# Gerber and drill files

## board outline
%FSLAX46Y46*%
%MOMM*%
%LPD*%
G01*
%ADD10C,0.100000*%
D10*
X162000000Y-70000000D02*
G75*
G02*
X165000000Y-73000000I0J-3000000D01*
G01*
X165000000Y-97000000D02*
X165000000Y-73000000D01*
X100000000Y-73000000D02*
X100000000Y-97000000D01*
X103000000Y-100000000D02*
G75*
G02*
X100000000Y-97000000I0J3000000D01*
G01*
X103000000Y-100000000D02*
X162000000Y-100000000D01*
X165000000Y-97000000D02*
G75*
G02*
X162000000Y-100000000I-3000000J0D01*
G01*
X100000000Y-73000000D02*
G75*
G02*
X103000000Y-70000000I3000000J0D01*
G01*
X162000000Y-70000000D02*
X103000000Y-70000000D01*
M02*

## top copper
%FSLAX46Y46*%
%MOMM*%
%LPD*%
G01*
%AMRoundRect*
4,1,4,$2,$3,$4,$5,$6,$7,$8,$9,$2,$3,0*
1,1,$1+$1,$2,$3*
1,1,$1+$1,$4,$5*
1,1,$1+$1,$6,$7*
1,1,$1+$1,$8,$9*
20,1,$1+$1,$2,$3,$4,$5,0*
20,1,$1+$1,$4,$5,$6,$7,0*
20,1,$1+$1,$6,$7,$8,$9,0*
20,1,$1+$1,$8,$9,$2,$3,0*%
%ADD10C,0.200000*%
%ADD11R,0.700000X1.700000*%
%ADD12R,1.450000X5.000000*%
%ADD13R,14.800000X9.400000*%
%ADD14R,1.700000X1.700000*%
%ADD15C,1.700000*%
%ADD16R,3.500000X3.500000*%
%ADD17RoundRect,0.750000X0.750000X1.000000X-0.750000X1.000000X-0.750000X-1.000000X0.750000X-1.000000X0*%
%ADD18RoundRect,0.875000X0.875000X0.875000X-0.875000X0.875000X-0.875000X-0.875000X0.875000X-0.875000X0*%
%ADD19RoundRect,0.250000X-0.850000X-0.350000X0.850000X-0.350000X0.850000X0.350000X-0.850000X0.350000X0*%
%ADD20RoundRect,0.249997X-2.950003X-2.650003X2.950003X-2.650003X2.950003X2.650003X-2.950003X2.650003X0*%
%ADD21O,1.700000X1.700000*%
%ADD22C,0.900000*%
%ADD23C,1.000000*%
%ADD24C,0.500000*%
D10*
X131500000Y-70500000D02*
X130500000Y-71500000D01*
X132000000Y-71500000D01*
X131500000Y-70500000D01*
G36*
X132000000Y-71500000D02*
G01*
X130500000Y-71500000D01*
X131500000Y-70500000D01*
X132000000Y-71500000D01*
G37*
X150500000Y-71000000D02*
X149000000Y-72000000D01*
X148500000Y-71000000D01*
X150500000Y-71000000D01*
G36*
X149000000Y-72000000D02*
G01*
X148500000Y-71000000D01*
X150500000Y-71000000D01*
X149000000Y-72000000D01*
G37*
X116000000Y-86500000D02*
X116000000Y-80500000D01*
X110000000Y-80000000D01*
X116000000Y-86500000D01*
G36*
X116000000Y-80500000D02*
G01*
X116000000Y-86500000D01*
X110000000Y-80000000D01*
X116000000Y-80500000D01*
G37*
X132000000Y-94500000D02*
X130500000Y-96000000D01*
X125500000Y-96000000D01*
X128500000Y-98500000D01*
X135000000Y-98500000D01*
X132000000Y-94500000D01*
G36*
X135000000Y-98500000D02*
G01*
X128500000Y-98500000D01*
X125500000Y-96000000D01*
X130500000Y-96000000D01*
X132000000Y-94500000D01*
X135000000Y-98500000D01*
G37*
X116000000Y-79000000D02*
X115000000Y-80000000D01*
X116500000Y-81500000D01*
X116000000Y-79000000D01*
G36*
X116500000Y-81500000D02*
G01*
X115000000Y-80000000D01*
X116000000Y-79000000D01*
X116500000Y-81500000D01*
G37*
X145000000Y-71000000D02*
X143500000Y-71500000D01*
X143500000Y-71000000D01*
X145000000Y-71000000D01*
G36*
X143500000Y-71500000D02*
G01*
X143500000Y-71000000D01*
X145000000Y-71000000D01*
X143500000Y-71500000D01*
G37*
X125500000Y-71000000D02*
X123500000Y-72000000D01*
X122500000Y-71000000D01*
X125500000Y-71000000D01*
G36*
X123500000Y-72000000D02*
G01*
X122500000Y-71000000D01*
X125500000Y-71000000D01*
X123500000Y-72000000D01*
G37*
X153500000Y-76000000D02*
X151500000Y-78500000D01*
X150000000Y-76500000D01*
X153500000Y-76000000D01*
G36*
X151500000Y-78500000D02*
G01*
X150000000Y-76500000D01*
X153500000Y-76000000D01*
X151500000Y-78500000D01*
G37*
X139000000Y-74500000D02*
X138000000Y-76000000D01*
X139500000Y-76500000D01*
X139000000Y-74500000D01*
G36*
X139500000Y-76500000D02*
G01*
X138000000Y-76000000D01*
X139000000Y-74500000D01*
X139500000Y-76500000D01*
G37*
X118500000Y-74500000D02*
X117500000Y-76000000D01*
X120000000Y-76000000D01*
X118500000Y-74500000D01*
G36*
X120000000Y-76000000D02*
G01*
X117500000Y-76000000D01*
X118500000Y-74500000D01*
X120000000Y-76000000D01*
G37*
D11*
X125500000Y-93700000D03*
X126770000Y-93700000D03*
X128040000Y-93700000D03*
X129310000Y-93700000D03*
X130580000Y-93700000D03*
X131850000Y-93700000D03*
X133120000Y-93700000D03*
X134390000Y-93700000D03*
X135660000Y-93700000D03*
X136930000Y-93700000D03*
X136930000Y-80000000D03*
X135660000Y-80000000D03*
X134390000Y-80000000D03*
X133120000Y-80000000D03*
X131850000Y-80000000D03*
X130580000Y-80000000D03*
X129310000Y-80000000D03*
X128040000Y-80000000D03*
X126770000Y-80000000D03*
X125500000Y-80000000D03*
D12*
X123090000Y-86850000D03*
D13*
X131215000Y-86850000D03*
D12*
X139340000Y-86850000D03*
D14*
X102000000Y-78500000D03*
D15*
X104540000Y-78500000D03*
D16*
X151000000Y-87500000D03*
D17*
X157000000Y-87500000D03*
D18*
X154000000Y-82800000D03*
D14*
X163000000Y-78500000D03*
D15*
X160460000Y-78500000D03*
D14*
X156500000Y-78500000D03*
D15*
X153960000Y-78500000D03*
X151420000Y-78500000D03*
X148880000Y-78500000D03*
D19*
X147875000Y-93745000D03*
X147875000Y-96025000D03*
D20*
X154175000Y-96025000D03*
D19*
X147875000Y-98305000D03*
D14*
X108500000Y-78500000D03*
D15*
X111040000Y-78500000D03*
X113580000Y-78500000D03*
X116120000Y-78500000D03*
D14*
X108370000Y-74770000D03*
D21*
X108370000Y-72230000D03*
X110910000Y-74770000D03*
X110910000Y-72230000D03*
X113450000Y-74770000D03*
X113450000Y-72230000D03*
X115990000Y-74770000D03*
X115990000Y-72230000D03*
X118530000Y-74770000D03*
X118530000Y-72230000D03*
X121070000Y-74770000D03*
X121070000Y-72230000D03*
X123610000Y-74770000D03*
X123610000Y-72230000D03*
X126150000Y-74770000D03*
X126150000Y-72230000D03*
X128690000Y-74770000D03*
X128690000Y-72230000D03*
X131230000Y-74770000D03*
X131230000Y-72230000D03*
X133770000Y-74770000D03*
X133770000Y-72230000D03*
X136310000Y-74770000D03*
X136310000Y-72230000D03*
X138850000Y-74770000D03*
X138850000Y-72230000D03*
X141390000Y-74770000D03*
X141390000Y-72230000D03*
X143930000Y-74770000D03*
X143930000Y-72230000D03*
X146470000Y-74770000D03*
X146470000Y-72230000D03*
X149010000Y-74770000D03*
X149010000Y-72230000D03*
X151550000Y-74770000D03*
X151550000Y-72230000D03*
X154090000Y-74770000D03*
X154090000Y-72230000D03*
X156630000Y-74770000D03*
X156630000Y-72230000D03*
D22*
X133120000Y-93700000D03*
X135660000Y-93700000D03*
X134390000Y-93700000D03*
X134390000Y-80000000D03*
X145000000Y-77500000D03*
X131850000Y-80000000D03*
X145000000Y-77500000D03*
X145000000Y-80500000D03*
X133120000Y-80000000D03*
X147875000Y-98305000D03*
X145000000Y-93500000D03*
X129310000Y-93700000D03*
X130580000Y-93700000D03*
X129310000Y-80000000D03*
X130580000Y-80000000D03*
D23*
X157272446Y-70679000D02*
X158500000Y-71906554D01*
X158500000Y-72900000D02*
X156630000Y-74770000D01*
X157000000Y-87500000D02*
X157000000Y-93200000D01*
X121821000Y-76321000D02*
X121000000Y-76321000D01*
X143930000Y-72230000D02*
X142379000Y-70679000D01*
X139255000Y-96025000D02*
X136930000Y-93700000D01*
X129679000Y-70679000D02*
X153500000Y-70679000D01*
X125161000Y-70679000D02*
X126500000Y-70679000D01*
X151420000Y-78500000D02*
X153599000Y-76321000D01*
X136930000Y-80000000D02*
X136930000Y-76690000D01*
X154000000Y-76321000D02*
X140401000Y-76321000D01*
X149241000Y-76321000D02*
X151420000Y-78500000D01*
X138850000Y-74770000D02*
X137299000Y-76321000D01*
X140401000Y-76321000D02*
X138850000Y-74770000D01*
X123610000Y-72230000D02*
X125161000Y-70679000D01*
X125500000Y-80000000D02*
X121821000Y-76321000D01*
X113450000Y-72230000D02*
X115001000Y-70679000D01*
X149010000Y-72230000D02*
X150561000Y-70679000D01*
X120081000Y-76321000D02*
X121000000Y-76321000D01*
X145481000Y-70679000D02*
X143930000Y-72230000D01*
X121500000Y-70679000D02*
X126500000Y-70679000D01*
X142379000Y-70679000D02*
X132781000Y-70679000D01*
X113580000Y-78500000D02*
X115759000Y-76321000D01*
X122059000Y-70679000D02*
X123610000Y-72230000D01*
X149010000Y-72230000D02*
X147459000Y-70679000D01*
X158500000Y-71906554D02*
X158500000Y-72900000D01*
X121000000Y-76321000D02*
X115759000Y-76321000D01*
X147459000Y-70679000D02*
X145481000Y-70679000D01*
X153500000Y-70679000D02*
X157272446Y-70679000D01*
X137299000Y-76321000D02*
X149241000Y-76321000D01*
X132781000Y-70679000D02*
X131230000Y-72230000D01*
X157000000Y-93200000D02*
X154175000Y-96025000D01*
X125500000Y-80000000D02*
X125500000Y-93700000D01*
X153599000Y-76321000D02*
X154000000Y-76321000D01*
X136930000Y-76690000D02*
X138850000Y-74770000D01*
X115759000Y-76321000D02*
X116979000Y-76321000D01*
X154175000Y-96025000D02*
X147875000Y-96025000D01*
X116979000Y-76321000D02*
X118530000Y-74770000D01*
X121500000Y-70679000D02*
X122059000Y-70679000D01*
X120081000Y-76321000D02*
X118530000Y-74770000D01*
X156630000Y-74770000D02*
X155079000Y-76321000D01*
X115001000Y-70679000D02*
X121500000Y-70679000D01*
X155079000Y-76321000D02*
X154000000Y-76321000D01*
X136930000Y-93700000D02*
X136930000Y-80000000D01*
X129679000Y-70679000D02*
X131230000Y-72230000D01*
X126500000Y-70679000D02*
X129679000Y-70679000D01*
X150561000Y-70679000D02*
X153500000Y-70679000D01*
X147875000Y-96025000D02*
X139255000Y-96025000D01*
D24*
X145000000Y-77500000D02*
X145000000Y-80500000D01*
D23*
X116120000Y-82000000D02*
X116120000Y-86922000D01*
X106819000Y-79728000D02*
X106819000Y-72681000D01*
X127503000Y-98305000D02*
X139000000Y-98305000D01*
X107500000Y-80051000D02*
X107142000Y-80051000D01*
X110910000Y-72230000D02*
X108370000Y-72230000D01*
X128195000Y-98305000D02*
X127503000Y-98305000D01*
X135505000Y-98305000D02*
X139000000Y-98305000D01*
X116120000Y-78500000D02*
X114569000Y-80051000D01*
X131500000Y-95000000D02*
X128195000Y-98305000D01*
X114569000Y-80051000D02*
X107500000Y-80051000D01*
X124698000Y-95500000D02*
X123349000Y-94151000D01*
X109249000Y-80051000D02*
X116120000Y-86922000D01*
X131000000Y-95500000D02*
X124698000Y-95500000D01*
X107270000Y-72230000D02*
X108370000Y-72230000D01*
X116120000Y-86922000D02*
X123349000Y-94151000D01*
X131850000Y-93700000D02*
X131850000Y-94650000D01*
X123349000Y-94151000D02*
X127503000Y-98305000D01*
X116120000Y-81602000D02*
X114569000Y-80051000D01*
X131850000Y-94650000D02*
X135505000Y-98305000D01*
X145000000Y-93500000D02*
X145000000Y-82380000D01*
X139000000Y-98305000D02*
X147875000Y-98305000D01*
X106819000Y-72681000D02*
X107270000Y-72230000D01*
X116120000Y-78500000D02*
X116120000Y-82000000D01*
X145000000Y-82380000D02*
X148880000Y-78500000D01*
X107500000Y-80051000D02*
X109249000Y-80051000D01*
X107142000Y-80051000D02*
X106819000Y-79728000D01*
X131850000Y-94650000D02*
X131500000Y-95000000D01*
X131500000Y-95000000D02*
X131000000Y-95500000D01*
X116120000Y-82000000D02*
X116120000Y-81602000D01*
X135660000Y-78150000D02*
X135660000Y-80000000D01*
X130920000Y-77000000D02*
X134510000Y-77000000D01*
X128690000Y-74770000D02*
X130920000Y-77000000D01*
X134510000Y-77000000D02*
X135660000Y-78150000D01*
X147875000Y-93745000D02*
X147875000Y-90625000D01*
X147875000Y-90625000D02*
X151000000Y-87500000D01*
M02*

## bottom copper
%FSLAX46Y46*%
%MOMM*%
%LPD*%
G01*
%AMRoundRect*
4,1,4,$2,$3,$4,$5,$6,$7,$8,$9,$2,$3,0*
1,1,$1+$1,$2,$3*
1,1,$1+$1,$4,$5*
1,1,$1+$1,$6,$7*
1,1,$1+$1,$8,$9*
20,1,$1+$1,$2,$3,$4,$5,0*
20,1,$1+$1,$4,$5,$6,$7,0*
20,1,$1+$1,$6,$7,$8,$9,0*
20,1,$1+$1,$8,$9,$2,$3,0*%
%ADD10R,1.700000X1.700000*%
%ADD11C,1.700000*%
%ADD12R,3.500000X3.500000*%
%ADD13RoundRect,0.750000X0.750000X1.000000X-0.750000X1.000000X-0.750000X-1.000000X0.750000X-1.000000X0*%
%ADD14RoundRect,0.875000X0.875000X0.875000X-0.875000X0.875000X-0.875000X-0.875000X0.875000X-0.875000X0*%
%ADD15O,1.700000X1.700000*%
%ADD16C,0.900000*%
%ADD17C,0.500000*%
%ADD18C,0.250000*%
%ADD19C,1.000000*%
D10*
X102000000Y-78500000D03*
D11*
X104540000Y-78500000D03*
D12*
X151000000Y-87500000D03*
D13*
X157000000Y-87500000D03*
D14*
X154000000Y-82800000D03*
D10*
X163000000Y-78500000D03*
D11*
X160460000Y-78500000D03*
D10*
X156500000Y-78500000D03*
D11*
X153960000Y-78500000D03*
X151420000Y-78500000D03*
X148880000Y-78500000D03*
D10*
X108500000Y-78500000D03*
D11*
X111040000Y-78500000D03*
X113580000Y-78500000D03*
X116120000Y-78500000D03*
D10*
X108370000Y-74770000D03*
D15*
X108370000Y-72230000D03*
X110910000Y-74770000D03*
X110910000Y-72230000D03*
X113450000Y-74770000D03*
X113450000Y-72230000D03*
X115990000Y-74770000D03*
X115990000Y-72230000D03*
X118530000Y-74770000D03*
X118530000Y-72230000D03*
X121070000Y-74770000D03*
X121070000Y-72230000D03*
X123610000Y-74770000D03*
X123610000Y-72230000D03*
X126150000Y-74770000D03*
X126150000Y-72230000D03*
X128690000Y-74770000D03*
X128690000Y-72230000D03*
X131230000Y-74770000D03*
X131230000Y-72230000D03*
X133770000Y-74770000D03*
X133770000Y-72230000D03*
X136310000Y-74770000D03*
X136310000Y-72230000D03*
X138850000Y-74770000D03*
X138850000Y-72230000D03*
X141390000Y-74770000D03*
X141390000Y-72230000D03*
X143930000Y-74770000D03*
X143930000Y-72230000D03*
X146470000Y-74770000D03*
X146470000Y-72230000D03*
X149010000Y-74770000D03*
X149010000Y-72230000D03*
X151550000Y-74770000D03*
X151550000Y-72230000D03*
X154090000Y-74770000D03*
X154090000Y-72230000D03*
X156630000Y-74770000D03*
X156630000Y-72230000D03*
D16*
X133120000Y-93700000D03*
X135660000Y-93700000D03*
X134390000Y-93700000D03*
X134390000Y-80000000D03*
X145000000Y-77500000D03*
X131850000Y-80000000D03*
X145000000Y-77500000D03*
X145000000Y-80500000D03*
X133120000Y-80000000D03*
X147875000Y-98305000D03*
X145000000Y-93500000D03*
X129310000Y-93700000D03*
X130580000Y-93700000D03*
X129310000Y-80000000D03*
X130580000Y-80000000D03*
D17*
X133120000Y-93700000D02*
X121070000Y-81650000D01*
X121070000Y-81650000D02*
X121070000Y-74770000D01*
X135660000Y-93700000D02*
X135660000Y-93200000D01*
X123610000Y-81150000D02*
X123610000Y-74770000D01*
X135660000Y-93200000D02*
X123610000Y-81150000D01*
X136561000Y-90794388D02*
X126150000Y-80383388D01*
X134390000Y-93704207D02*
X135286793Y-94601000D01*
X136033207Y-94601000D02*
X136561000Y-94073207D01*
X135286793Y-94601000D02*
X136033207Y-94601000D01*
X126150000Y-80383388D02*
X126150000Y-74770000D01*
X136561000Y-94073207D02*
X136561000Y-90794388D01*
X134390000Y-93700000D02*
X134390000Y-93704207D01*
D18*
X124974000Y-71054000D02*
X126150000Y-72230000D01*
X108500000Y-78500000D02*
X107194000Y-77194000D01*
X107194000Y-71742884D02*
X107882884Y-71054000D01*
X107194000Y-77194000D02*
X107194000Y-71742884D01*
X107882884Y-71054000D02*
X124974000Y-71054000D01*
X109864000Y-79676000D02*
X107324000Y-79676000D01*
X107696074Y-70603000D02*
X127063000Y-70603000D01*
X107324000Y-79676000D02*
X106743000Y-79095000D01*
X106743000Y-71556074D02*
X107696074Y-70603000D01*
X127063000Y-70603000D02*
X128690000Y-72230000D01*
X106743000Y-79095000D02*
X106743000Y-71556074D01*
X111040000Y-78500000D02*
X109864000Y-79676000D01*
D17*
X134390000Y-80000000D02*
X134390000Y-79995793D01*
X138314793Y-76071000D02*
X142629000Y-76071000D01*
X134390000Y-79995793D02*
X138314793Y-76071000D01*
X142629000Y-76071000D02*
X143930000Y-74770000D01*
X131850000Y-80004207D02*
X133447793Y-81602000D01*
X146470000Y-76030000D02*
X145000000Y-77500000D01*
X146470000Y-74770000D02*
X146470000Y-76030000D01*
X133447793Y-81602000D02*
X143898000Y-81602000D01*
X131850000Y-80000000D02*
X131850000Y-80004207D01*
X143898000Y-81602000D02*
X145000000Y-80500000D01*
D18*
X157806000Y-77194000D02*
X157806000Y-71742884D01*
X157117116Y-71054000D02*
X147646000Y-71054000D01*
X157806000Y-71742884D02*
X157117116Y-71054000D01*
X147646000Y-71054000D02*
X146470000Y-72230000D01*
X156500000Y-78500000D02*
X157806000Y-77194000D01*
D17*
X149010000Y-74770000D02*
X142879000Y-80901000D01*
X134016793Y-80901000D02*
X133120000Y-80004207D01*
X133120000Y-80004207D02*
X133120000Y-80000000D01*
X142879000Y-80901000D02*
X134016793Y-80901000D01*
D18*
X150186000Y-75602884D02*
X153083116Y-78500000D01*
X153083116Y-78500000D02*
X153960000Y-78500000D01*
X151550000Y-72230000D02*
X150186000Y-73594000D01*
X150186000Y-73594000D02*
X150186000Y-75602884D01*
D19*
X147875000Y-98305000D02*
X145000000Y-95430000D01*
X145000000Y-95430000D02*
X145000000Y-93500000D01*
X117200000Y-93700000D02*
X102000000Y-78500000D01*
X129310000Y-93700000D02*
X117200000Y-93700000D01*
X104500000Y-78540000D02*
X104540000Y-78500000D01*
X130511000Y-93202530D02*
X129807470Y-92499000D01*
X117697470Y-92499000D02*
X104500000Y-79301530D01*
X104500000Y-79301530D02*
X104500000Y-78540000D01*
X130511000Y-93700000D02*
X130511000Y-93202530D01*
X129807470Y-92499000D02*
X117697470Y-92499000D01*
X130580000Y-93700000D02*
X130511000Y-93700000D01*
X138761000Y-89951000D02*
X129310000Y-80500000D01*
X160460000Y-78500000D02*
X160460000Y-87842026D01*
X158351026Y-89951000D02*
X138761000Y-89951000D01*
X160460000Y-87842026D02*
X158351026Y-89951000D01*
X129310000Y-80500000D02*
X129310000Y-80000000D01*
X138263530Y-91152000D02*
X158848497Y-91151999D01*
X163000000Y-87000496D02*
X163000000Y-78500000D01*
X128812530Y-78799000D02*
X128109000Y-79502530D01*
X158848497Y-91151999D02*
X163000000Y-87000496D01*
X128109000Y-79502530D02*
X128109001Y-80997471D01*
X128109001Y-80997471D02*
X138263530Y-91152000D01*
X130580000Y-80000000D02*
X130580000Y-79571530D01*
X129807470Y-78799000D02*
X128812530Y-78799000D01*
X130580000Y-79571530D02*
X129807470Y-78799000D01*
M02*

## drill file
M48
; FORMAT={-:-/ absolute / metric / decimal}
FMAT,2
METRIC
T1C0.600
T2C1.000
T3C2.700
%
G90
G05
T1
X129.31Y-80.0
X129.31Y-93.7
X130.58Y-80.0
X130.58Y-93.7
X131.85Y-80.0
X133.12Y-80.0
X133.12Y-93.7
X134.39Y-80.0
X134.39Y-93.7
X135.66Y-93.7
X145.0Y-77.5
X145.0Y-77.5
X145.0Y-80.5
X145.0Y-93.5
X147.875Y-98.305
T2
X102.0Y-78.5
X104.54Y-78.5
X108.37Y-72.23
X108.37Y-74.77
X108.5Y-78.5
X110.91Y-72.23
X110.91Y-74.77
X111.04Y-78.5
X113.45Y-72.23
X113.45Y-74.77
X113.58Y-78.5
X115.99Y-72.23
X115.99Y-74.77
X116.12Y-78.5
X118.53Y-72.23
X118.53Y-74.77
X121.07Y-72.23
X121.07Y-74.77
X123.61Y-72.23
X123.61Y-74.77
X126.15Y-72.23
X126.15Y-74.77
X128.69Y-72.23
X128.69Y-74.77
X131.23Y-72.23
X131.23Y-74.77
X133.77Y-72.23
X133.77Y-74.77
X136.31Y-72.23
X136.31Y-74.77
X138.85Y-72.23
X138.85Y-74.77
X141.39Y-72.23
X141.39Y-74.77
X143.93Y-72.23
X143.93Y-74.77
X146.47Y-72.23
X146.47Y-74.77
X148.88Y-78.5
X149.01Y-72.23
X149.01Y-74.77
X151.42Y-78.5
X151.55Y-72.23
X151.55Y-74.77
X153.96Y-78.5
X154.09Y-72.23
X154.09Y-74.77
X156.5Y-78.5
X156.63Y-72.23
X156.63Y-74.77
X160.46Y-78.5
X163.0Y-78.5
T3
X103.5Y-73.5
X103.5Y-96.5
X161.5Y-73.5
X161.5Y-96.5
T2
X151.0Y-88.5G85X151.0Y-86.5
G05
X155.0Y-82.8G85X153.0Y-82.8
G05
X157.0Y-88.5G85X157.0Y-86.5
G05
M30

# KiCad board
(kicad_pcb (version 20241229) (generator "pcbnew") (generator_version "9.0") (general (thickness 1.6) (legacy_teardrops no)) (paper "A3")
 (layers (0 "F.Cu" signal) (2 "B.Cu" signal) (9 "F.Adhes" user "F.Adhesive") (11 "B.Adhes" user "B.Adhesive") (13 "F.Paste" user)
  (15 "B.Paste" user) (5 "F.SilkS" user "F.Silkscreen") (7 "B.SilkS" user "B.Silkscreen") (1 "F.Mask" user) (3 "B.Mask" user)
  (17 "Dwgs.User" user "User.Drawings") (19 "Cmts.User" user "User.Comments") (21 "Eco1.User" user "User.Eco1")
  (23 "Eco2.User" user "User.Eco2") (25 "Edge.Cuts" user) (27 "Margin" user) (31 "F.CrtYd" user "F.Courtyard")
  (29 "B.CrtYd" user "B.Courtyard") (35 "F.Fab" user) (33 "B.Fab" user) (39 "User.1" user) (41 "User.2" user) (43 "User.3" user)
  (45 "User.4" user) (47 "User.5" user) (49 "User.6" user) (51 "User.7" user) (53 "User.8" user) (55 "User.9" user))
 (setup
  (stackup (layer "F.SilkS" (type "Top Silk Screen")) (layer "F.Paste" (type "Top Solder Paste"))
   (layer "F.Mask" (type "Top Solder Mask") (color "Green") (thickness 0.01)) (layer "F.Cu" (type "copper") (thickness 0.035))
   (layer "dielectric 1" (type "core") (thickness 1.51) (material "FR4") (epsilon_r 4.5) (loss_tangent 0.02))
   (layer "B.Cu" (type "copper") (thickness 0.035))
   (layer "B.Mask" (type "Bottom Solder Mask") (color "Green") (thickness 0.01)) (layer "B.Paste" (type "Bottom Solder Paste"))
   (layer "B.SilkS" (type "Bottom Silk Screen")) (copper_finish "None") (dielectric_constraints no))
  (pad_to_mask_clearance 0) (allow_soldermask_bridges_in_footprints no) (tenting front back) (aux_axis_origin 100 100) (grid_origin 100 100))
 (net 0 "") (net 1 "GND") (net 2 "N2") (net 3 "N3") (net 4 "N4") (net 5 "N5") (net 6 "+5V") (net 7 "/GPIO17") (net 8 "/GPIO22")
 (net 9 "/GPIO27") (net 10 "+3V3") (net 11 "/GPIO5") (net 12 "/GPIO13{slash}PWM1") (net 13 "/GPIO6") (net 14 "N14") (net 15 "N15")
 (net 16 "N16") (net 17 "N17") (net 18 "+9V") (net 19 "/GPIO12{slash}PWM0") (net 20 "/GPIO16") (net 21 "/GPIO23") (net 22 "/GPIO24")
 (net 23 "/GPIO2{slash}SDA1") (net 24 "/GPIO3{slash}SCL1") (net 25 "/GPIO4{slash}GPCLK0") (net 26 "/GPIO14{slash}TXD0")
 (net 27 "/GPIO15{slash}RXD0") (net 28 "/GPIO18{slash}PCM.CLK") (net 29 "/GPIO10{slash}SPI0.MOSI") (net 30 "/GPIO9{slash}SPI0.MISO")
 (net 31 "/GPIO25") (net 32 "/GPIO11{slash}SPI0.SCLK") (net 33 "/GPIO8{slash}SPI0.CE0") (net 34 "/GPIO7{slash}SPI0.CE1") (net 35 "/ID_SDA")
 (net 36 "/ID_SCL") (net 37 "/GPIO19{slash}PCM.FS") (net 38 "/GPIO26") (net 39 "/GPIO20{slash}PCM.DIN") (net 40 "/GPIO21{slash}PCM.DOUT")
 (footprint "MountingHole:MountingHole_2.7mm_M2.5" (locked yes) (layer "F.Cu") (at 161.5 73.5)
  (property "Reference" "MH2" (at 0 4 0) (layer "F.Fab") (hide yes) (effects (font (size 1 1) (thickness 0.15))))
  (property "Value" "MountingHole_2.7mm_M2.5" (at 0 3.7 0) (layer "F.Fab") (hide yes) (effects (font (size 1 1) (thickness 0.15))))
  (pad "" np_thru_hole circle (at 0 0) (size 2.7 2.7) (drill 2.7) (layers "*.Cu" "*.Mask")))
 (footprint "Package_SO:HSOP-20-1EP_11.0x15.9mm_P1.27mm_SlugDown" (layer "F.Cu") (at 131.215 86.85 90)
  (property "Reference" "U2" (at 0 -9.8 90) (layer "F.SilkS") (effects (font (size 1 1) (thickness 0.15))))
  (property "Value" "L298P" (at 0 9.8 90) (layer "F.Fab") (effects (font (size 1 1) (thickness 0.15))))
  (pad "1" smd rect (at -6.85 -5.715 90) (size 1.7 0.7) (layers "F.Cu" "F.Mask" "F.Paste") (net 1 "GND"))
  (pad "2" smd rect (at -6.85 -4.445 90) (size 1.7 0.7) (layers "F.Cu" "F.Mask" "F.Paste") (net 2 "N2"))
  (pad "3" smd rect (at -6.85 -3.175 90) (size 1.7 0.7) (layers "F.Cu" "F.Mask" "F.Paste") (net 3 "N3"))
  (pad "4" smd rect (at -6.85 -1.905 90) (size 1.7 0.7) (layers "F.Cu" "F.Mask" "F.Paste") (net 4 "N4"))
  (pad "5" smd rect (at -6.85 -0.635 90) (size 1.7 0.7) (layers "F.Cu" "F.Mask" "F.Paste") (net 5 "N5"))
  (pad "6" smd rect (at -6.85 0.635 90) (size 1.7 0.7) (layers "F.Cu" "F.Mask" "F.Paste") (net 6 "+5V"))
  (pad "7" smd rect (at -6.85 1.905 90) (size 1.7 0.7) (layers "F.Cu" "F.Mask" "F.Paste") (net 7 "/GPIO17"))
  (pad "8" smd rect (at -6.85 3.175 90) (size 1.7 0.7) (layers "F.Cu" "F.Mask" "F.Paste") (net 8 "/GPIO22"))
  (pad "9" smd rect (at -6.85 4.445 90) (size 1.7 0.7) (layers "F.Cu" "F.Mask" "F.Paste") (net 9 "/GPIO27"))
  (pad "10" smd rect (at -6.85 5.715 90) (size 1.7 0.7) (layers "F.Cu" "F.Mask" "F.Paste") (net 1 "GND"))
  (pad "11" smd rect (at 6.85 5.715 90) (size 1.7 0.7) (layers "F.Cu" "F.Mask" "F.Paste") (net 1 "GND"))
  (pad "12" smd rect (at 6.85 4.445 90) (size 1.7 0.7) (layers "F.Cu" "F.Mask" "F.Paste") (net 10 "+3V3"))
  (pad "13" smd rect (at 6.85 3.175 90) (size 1.7 0.7) (layers "F.Cu" "F.Mask" "F.Paste") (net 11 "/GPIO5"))
  (pad "14" smd rect (at 6.85 1.905 90) (size 1.7 0.7) (layers "F.Cu" "F.Mask" "F.Paste") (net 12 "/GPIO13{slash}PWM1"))
  (pad "15" smd rect (at 6.85 0.635 90) (size 1.7 0.7) (layers "F.Cu" "F.Mask" "F.Paste") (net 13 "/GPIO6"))
  (pad "16" smd rect (at 6.85 -0.635 90) (size 1.7 0.7) (layers "F.Cu" "F.Mask" "F.Paste") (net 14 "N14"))
  (pad "17" smd rect (at 6.85 -1.905 90) (size 1.7 0.7) (layers "F.Cu" "F.Mask" "F.Paste") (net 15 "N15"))
  (pad "18" smd rect (at 6.85 -3.175 90) (size 1.7 0.7) (layers "F.Cu" "F.Mask" "F.Paste") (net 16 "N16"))
  (pad "19" smd rect (at 6.85 -4.445 90) (size 1.7 0.7) (layers "F.Cu" "F.Mask" "F.Paste") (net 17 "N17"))
  (pad "20" smd rect (at 6.85 -5.715 90) (size 1.7 0.7) (layers "F.Cu" "F.Mask" "F.Paste") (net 1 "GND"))
  (pad "21" smd rect (at 0 -8.125 90) (size 5 1.45) (layers "F.Cu" "F.Mask" "F.Paste") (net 1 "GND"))
  (pad "21" smd rect (at 0 0 90) (size 9.4 14.8) (layers "F.Cu" "F.Mask" "F.Paste") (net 1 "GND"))
  (pad "21" smd rect (at 0 8.125 90) (size 5 1.45) (layers "F.Cu" "F.Mask" "F.Paste") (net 1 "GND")))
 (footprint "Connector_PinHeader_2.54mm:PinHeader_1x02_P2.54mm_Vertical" (layer "F.Cu") (at 102 78.5 90)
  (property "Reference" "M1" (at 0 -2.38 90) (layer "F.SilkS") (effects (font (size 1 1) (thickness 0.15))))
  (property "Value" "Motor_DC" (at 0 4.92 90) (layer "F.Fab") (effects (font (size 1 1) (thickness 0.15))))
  (pad "1" thru_hole rect (at 0 0 90) (size 1.7 1.7) (drill 1) (layers "*.Cu" "*.Mask") (remove_unused_layers no) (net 4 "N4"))
  (pad "2" thru_hole circle (at 0 2.54 90) (size 1.7 1.7) (drill 1) (layers "*.Cu" "*.Mask") (remove_unused_layers no) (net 5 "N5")))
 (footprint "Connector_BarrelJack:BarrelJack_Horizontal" (layer "F.Cu") (at 151 87.5 180)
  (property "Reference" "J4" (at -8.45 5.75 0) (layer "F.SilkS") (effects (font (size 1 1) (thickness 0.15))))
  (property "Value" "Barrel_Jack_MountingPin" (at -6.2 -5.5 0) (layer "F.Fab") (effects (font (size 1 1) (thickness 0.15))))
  (pad "1" thru_hole rect (at 0 0 180) (size 3.5 3.5) (drill oval 1 3) (layers "*.Cu" "*.Mask") (remove_unused_layers no) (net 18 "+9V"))
  (pad "2" thru_hole roundrect (at -6 0 180) (size 3 3.5) (drill oval 1 3) (layers "*.Cu" "*.Mask") (remove_unused_layers no)
   (roundrect_rratio 0.25) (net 1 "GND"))
  (pad "3" thru_hole roundrect (at -3 4.7 180) (size 3.5 3.5) (drill oval 3 1) (layers "*.Cu" "*.Mask") (remove_unused_layers no)
   (roundrect_rratio 0.25)))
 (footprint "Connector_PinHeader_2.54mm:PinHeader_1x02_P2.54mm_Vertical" (layer "F.Cu") (at 163 78.5 -90)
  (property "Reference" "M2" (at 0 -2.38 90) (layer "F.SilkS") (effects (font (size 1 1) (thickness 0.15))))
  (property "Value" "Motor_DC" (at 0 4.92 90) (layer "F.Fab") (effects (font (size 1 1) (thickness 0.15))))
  (pad "1" thru_hole rect (at 0 0 270) (size 1.7 1.7) (drill 1) (layers "*.Cu" "*.Mask") (remove_unused_layers no) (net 14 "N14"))
  (pad "2" thru_hole circle (at 0 2.54 270) (size 1.7 1.7) (drill 1) (layers "*.Cu" "*.Mask") (remove_unused_layers no) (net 15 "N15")))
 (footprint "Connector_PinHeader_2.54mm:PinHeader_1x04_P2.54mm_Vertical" (layer "F.Cu") (at 156.5 78.5 -90)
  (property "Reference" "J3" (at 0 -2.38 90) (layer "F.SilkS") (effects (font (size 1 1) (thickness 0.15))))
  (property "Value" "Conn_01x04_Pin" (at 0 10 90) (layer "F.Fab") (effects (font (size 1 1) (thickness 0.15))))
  (pad "1" thru_hole rect (at 0 0 270) (size 1.7 1.7) (drill 1) (layers "*.Cu" "*.Mask") (remove_unused_layers no)
   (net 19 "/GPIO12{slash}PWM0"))
  (pad "2" thru_hole circle (at 0 2.54 270) (size 1.7 1.7) (drill 1) (layers "*.Cu" "*.Mask") (remove_unused_layers no) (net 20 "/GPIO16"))
  (pad "3" thru_hole circle (at 0 5.08 270) (size 1.7 1.7) (drill 1) (layers "*.Cu" "*.Mask") (remove_unused_layers no) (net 1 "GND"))
  (pad "4" thru_hole circle (at 0 7.62 270) (size 1.7 1.7) (drill 1) (layers "*.Cu" "*.Mask") (remove_unused_layers no) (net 6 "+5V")))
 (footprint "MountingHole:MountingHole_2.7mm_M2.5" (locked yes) (layer "F.Cu") (at 103.5 96.5)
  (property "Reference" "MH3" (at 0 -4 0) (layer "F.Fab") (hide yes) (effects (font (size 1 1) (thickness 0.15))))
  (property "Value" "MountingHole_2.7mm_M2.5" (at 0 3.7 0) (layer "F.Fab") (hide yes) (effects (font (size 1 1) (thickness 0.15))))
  (pad "" np_thru_hole circle (at 0 0) (size 2.7 2.7) (drill 2.7) (layers "*.Cu" "*.Mask")))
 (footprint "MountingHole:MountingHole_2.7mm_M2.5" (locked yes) (layer "F.Cu") (at 103.5 73.5)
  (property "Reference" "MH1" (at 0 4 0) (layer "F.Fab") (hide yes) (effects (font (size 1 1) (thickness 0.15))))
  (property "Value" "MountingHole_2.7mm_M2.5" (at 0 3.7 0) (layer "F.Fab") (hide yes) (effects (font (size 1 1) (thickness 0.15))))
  (pad "" np_thru_hole circle (at 0 0) (size 2.7 2.7) (drill 2.7) (layers "*.Cu" "*.Mask")))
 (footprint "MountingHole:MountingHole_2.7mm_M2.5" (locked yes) (layer "F.Cu") (at 161.5 96.5)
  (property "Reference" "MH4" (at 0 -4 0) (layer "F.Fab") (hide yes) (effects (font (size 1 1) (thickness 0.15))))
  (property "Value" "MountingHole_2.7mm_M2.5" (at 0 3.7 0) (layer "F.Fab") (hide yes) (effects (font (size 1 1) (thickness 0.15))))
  (pad "" np_thru_hole circle (at 0 0) (size 2.7 2.7) (drill 2.7) (layers "*.Cu" "*.Mask")))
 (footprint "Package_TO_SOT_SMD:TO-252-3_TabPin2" (layer "F.Cu") (at 152.915 96.025)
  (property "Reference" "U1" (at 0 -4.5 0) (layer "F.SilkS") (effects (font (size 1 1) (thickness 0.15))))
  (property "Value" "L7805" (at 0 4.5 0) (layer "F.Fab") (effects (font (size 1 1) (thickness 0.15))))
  (pad "" smd roundrect (at -0.415 -1.525) (size 3.05 2.75) (layers "F.Paste") (roundrect_rratio 0.090909))
  (pad "" smd roundrect (at -0.415 1.525) (size 3.05 2.75) (layers "F.Paste") (roundrect_rratio 0.090909))
  (pad "" smd roundrect (at 2.935 -1.525) (size 3.05 2.75) (layers "F.Paste") (roundrect_rratio 0.090909))
  (pad "" smd roundrect (at 2.935 1.525) (size 3.05 2.75) (layers "F.Paste") (roundrect_rratio 0.090909))
  (pad "1" smd roundrect (at -5.04 -2.28) (size 2.2 1.2) (layers "F.Cu" "F.Mask" "F.Paste") (roundrect_rratio 0.208333) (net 18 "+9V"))
  (pad "2" smd roundrect (at -5.04 0) (size 2.2 1.2) (layers "F.Cu" "F.Mask" "F.Paste") (roundrect_rratio 0.208333) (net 1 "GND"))
  (pad "2" smd roundrect (at 1.26 0) (size 6.4 5.8) (layers "F.Cu" "F.Mask") (roundrect_rratio 0.043103) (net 1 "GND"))
  (pad "3" smd roundrect (at -5.04 2.28) (size 2.2 1.2) (layers "F.Cu" "F.Mask" "F.Paste") (roundrect_rratio 0.208333) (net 6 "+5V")))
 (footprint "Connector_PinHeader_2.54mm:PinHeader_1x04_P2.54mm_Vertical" (layer "F.Cu") (at 108.5 78.5 90)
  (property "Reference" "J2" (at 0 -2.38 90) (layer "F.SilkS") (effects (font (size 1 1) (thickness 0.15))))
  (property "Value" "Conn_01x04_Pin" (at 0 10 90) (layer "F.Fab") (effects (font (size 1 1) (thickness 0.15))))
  (pad "1" thru_hole rect (at 0 0 90) (size 1.7 1.7) (drill 1) (layers "*.Cu" "*.Mask") (remove_unused_layers no) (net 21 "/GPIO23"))
  (pad "2" thru_hole circle (at 0 2.54 90) (size 1.7 1.7) (drill 1) (layers "*.Cu" "*.Mask") (remove_unused_layers no) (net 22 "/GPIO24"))
  (pad "3" thru_hole circle (at 0 5.08 90) (size 1.7 1.7) (drill 1) (layers "*.Cu" "*.Mask") (remove_unused_layers no) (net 1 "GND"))
  (pad "4" thru_hole circle (at 0 7.62 90) (size 1.7 1.7) (drill 1) (layers "*.Cu" "*.Mask") (remove_unused_layers no) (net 6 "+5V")))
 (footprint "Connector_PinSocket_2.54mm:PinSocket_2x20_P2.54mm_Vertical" (layer "B.Cu") (at 108.37 74.77 -90)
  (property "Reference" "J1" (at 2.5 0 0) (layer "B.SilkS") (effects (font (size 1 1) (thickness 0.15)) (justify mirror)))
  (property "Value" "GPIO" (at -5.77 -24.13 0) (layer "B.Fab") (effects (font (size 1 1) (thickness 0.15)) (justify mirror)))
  (pad "1" thru_hole rect (at 0 0 270) (size 1.7 1.7) (drill 1) (layers "*.Cu" "*.Mask") (remove_unused_layers no) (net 10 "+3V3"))
  (pad "2" thru_hole oval (at -2.54 0 270) (size 1.7 1.7) (drill 1) (layers "*.Cu" "*.Mask") (remove_unused_layers no) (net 6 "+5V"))
  (pad "3" thru_hole oval (at 0 -2.54 270) (size 1.7 1.7) (drill 1) (layers "*.Cu" "*.Mask") (remove_unused_layers no)
   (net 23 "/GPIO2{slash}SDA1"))
  (pad "4" thru_hole oval (at -2.54 -2.54 270) (size 1.7 1.7) (drill 1) (layers "*.Cu" "*.Mask") (remove_unused_layers no) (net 6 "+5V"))
  (pad "5" thru_hole oval (at 0 -5.08 270) (size 1.7 1.7) (drill 1) (layers "*.Cu" "*.Mask") (remove_unused_layers no)
   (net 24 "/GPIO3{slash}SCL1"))
  (pad "6" thru_hole oval (at -2.54 -5.08 270) (size 1.7 1.7) (drill 1) (layers "*.Cu" "*.Mask") (remove_unused_layers no) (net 1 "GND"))
  (pad "7" thru_hole oval (at 0 -7.62 270) (size 1.7 1.7) (drill 1) (layers "*.Cu" "*.Mask") (remove_unused_layers no)
   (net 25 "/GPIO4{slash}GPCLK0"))
  (pad "8" thru_hole oval (at -2.54 -7.62 270) (size 1.7 1.7) (drill 1) (layers "*.Cu" "*.Mask") (remove_unused_layers no)
   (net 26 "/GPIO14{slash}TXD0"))
  (pad "9" thru_hole oval (at 0 -10.16 270) (size 1.7 1.7) (drill 1) (layers "*.Cu" "*.Mask") (remove_unused_layers no) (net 1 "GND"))
  (pad "10" thru_hole oval (at -2.54 -10.16 270) (size 1.7 1.7) (drill 1) (layers "*.Cu" "*.Mask") (remove_unused_layers no)
   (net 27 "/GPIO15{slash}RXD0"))
  (pad "11" thru_hole oval (at 0 -12.7 270) (size 1.7 1.7) (drill 1) (layers "*.Cu" "*.Mask") (remove_unused_layers no) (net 7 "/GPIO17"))
  (pad "12" thru_hole oval (at -2.54 -12.7 270) (size 1.7 1.7) (drill 1) (layers "*.Cu" "*.Mask") (remove_unused_layers no)
   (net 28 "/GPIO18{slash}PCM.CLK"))
  (pad "13" thru_hole oval (at 0 -15.24 270) (size 1.7 1.7) (drill 1) (layers "*.Cu" "*.Mask") (remove_unused_layers no) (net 9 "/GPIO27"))
  (pad "14" thru_hole oval (at -2.54 -15.24 270) (size 1.7 1.7) (drill 1) (layers "*.Cu" "*.Mask") (remove_unused_layers no) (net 1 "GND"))
  (pad "15" thru_hole oval (at 0 -17.78 270) (size 1.7 1.7) (drill 1) (layers "*.Cu" "*.Mask") (remove_unused_layers no) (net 8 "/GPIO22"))
  (pad "16" thru_hole oval (at -2.54 -17.78 270) (size 1.7 1.7) (drill 1) (layers "*.Cu" "*.Mask") (remove_unused_layers no)
   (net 21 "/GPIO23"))
  (pad "17" thru_hole oval (at 0 -20.32 270) (size 1.7 1.7) (drill 1) (layers "*.Cu" "*.Mask") (remove_unused_layers no) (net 10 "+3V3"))
  (pad "18" thru_hole oval (at -2.54 -20.32 270) (size 1.7 1.7) (drill 1) (layers "*.Cu" "*.Mask") (remove_unused_layers no)
   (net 22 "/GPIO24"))
  (pad "19" thru_hole oval (at 0 -22.86 270) (size 1.7 1.7) (drill 1) (layers "*.Cu" "*.Mask") (remove_unused_layers no)
   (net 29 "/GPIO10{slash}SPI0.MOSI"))
  (pad "20" thru_hole oval (at -2.54 -22.86 270) (size 1.7 1.7) (drill 1) (layers "*.Cu" "*.Mask") (remove_unused_layers no) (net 1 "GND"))
  (pad "21" thru_hole oval (at 0 -25.4 270) (size 1.7 1.7) (drill 1) (layers "*.Cu" "*.Mask") (remove_unused_layers no)
   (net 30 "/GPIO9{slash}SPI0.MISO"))
  (pad "22" thru_hole oval (at -2.54 -25.4 270) (size 1.7 1.7) (drill 1) (layers "*.Cu" "*.Mask") (remove_unused_layers no)
   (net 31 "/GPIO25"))
  (pad "23" thru_hole oval (at 0 -27.94 270) (size 1.7 1.7) (drill 1) (layers "*.Cu" "*.Mask") (remove_unused_layers no)
   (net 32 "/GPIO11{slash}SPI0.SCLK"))
  (pad "24" thru_hole oval (at -2.54 -27.94 270) (size 1.7 1.7) (drill 1) (layers "*.Cu" "*.Mask") (remove_unused_layers no)
   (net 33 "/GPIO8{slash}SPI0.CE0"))
  (pad "25" thru_hole oval (at 0 -30.48 270) (size 1.7 1.7) (drill 1) (layers "*.Cu" "*.Mask") (remove_unused_layers no) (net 1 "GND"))
  (pad "26" thru_hole oval (at -2.54 -30.48 270) (size 1.7 1.7) (drill 1) (layers "*.Cu" "*.Mask") (remove_unused_layers no)
   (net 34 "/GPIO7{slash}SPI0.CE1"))
  (pad "27" thru_hole oval (at 0 -33.02 270) (size 1.7 1.7) (drill 1) (layers "*.Cu" "*.Mask") (remove_unused_layers no) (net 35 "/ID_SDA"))
  (pad "28" thru_hole oval (at -2.54 -33.02 270) (size 1.7 1.7) (drill 1) (layers "*.Cu" "*.Mask") (remove_unused_layers no)
   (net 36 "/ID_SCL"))
  (pad "29" thru_hole oval (at 0 -35.56 270) (size 1.7 1.7) (drill 1) (layers "*.Cu" "*.Mask") (remove_unused_layers no) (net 11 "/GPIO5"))
  (pad "30" thru_hole oval (at -2.54 -35.56 270) (size 1.7 1.7) (drill 1) (layers "*.Cu" "*.Mask") (remove_unused_layers no) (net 1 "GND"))
  (pad "31" thru_hole oval (at 0 -38.1 270) (size 1.7 1.7) (drill 1) (layers "*.Cu" "*.Mask") (remove_unused_layers no) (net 13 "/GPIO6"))
  (pad "32" thru_hole oval (at -2.54 -38.1 270) (size 1.7 1.7) (drill 1) (layers "*.Cu" "*.Mask") (remove_unused_layers no)
   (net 19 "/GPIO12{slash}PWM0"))
  (pad "33" thru_hole oval (at 0 -40.64 270) (size 1.7 1.7) (drill 1) (layers "*.Cu" "*.Mask") (remove_unused_layers no)
   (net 12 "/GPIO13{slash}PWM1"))
  (pad "34" thru_hole oval (at -2.54 -40.64 270) (size 1.7 1.7) (drill 1) (layers "*.Cu" "*.Mask") (remove_unused_layers no) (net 1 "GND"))
  (pad "35" thru_hole oval (at 0 -43.18 270) (size 1.7 1.7) (drill 1) (layers "*.Cu" "*.Mask") (remove_unused_layers no)
   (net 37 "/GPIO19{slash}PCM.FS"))
  (pad "36" thru_hole oval (at -2.54 -43.18 270) (size 1.7 1.7) (drill 1) (layers "*.Cu" "*.Mask") (remove_unused_layers no)
   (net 20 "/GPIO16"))
  (pad "37" thru_hole oval (at 0 -45.72 270) (size 1.7 1.7) (drill 1) (layers "*.Cu" "*.Mask") (remove_unused_layers no) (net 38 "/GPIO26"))
  (pad "38" thru_hole oval (at -2.54 -45.72 270) (size 1.7 1.7) (drill 1) (layers "*.Cu" "*.Mask") (remove_unused_layers no)
   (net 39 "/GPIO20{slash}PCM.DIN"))
  (pad "39" thru_hole oval (at 0 -48.26 270) (size 1.7 1.7) (drill 1) (layers "*.Cu" "*.Mask") (remove_unused_layers no) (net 1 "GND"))
  (pad "40" thru_hole oval (at -2.54 -48.26 270) (size 1.7 1.7) (drill 1) (layers "*.Cu" "*.Mask") (remove_unused_layers no)
   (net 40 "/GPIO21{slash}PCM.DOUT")))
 (gr_poly (pts (xy 131.5 70.5) (xy 130.5 71.5) (xy 132 71.5)) (stroke (width 0.2) (type solid)) (fill yes) (layer "F.Cu") (net 1))
 (gr_poly (pts (xy 150.5 71) (xy 149 72) (xy 148.5 71)) (stroke (width 0.2) (type solid)) (fill yes) (layer "F.Cu") (net 1))
 (gr_poly (pts (xy 116 86.5) (xy 116 80.5) (xy 110 80)) (stroke (width 0.2) (type solid)) (fill yes) (layer "F.Cu") (net 6))
 (gr_poly
  (pts (xy 132 94.5) (xy 130.5 96) (xy 125.5 96) (xy 128.5 98.5) (xy 135 98.5)) (stroke (width 0.2) (type solid)) (fill yes) (layer "F.Cu")
  (net 6))
 (gr_poly (pts (xy 116 79) (xy 115 80) (xy 116.5 81.5)) (stroke (width 0.2) (type solid)) (fill yes) (layer "F.Cu") (net 6))
 (gr_poly (pts (xy 145 71) (xy 143.5 71.5) (xy 143.5 71)) (stroke (width 0.2) (type solid)) (fill yes) (layer "F.Cu") (net 1))
 (gr_poly (pts (xy 125.5 71) (xy 123.5 72) (xy 122.5 71)) (stroke (width 0.2) (type solid)) (fill yes) (layer "F.Cu") (net 1))
 (gr_poly (pts (xy 153.5 76) (xy 151.5 78.5) (xy 150 76.5)) (stroke (width 0.2) (type solid)) (fill yes) (layer "F.Cu") (net 1))
 (gr_poly (pts (xy 139 74.5) (xy 138 76) (xy 139.5 76.5)) (stroke (width 0.2) (type solid)) (fill yes) (layer "F.Cu") (net 1))
 (gr_poly (pts (xy 118.5 74.5) (xy 117.5 76) (xy 120 76)) (stroke (width 0.2) (type solid)) (fill yes) (layer "F.Cu") (net 1))
 (gr_arc (start 162 70) (mid 164.12132 70.87868) (end 165 73) (stroke (width 0.1) (type solid)) (layer "Edge.Cuts"))
 (gr_line (start 165 97) (end 165 73) (stroke (width 0.1) (type solid)) (layer "Edge.Cuts"))
 (gr_line (start 100 73) (end 100 97) (stroke (width 0.1) (type solid)) (layer "Edge.Cuts"))
 (gr_arc (start 103 100) (mid 100.87868 99.12132) (end 100 97) (stroke (width 0.1) (type solid)) (layer "Edge.Cuts"))
 (gr_line (start 103 100) (end 162 100) (stroke (width 0.1) (type solid)) (layer "Edge.Cuts"))
 (gr_arc (start 165 97) (mid 164.12132 99.12132) (end 162 100) (stroke (width 0.1) (type solid)) (layer "Edge.Cuts"))
 (gr_arc (start 100 73) (mid 100.87868 70.87868) (end 103 70) (stroke (width 0.1) (type solid)) (layer "Edge.Cuts"))
 (gr_line (start 162 70) (end 103 70) (stroke (width 0.1) (type solid)) (layer "Edge.Cuts"))
 (segment (start 157.272446 70.679) (end 158.5 71.906554) (width 1) (layer "F.Cu") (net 1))
 (segment (start 158.5 72.9) (end 156.63 74.77) (width 1) (layer "F.Cu") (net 1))
 (segment (start 157 87.5) (end 157 93.2) (width 1) (layer "F.Cu") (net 1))
 (segment (start 121.821 76.321) (end 121 76.321) (width 1) (layer "F.Cu") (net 1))
 (segment (start 143.93 72.23) (end 142.379 70.679) (width 1) (layer "F.Cu") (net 1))
 (segment (start 139.255 96.025) (end 136.93 93.7) (width 1) (layer "F.Cu") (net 1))
 (segment (start 129.679 70.679) (end 153.5 70.679) (width 1) (layer "F.Cu") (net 1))
 (segment (start 125.161 70.679) (end 126.5 70.679) (width 1) (layer "F.Cu") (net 1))
 (segment (start 151.42 78.5) (end 153.599 76.321) (width 1) (layer "F.Cu") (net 1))
 (segment (start 136.93 80) (end 136.93 76.69) (width 1) (layer "F.Cu") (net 1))
 (segment (start 154 76.321) (end 140.401 76.321) (width 1) (layer "F.Cu") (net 1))
 (segment (start 149.241 76.321) (end 151.42 78.5) (width 1) (layer "F.Cu") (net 1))
 (segment (start 138.85 74.77) (end 137.299 76.321) (width 1) (layer "F.Cu") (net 1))
 (segment (start 140.401 76.321) (end 138.85 74.77) (width 1) (layer "F.Cu") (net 1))
 (segment (start 123.61 72.23) (end 125.161 70.679) (width 1) (layer "F.Cu") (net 1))
 (segment (start 125.5 80) (end 121.821 76.321) (width 1) (layer "F.Cu") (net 1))
 (segment (start 113.45 72.23) (end 115.001 70.679) (width 1) (layer "F.Cu") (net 1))
 (segment (start 149.01 72.23) (end 150.561 70.679) (width 1) (layer "F.Cu") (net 1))
 (segment (start 120.081 76.321) (end 121 76.321) (width 1) (layer "F.Cu") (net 1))
 (segment (start 145.481 70.679) (end 143.93 72.23) (width 1) (layer "F.Cu") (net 1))
 (segment (start 121.5 70.679) (end 126.5 70.679) (width 1) (layer "F.Cu") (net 1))
 (segment (start 142.379 70.679) (end 132.781 70.679) (width 1) (layer "F.Cu") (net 1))
 (segment (start 113.58 78.5) (end 115.759 76.321) (width 1) (layer "F.Cu") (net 1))
 (segment (start 122.059 70.679) (end 123.61 72.23) (width 1) (layer "F.Cu") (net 1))
 (segment (start 149.01 72.23) (end 147.459 70.679) (width 1) (layer "F.Cu") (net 1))
 (segment (start 158.5 71.906554) (end 158.5 72.9) (width 1) (layer "F.Cu") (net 1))
 (segment (start 121 76.321) (end 115.759 76.321) (width 1) (layer "F.Cu") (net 1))
 (segment (start 147.459 70.679) (end 145.481 70.679) (width 1) (layer "F.Cu") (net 1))
 (segment (start 153.5 70.679) (end 157.272446 70.679) (width 1) (layer "F.Cu") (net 1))
 (segment (start 137.299 76.321) (end 149.241 76.321) (width 1) (layer "F.Cu") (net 1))
 (segment (start 132.781 70.679) (end 131.23 72.23) (width 1) (layer "F.Cu") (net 1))
 (segment (start 157 93.2) (end 154.175 96.025) (width 1) (layer "F.Cu") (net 1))
 (segment (start 125.5 80) (end 125.5 93.7) (width 1) (layer "F.Cu") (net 1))
 (segment (start 153.599 76.321) (end 154 76.321) (width 1) (layer "F.Cu") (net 1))
 (segment (start 136.93 76.69) (end 138.85 74.77) (width 1) (layer "F.Cu") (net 1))
 (segment (start 115.759 76.321) (end 116.979 76.321) (width 1) (layer "F.Cu") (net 1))
 (segment (start 154.175 96.025) (end 147.875 96.025) (width 1) (layer "F.Cu") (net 1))
 (segment (start 116.979 76.321) (end 118.53 74.77) (width 1) (layer "F.Cu") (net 1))
 (segment (start 121.5 70.679) (end 122.059 70.679) (width 1) (layer "F.Cu") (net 1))
 (segment (start 120.081 76.321) (end 118.53 74.77) (width 1) (layer "F.Cu") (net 1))
 (segment (start 156.63 74.77) (end 155.079 76.321) (width 1) (layer "F.Cu") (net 1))
 (segment (start 115.001 70.679) (end 121.5 70.679) (width 1) (layer "F.Cu") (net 1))
 (segment (start 155.079 76.321) (end 154 76.321) (width 1) (layer "F.Cu") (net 1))
 (segment (start 136.93 93.7) (end 136.93 80) (width 1) (layer "F.Cu") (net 1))
 (segment (start 129.679 70.679) (end 131.23 72.23) (width 1) (layer "F.Cu") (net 1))
 (segment (start 126.5 70.679) (end 129.679 70.679) (width 1) (layer "F.Cu") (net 1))
 (segment (start 150.561 70.679) (end 153.5 70.679) (width 1) (layer "F.Cu") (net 1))
 (segment (start 147.875 96.025) (end 139.255 96.025) (width 1) (layer "F.Cu") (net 1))
 (via (at 133.12 93.7) (size 0.9) (drill 0.6) (layers "F.Cu" "B.Cu") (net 7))
 (segment (start 133.12 93.7) (end 121.07 81.65) (width 0.5) (layer "B.Cu") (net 7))
 (segment (start 121.07 81.65) (end 121.07 74.77) (width 0.5) (layer "B.Cu") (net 7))
 (via (at 135.66 93.7) (size 0.9) (drill 0.6) (layers "F.Cu" "B.Cu") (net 9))
 (segment (start 135.66 93.7) (end 135.66 93.2) (width 0.5) (layer "B.Cu") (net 9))
 (segment (start 123.61 81.15) (end 123.61 74.77) (width 0.5) (layer "B.Cu") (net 9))
 (segment (start 135.66 93.2) (end 123.61 81.15) (width 0.5) (layer "B.Cu") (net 9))
 (via (at 134.39 93.7) (size 0.9) (drill 0.6) (layers "F.Cu" "B.Cu") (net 8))
 (segment (start 136.561 90.794388) (end 126.15 80.383388) (width 0.5) (layer "B.Cu") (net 8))
 (segment (start 134.39 93.704207) (end 135.286793 94.601) (width 0.5) (layer "B.Cu") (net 8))
 (segment (start 136.033207 94.601) (end 136.561 94.073207) (width 0.5) (layer "B.Cu") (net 8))
 (segment (start 135.286793 94.601) (end 136.033207 94.601) (width 0.5) (layer "B.Cu") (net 8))
 (segment (start 126.15 80.383388) (end 126.15 74.77) (width 0.5) (layer "B.Cu") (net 8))
 (segment (start 136.561 94.073207) (end 136.561 90.794388) (width 0.5) (layer "B.Cu") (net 8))
 (segment (start 134.39 93.7) (end 134.39 93.704207) (width 0.5) (layer "B.Cu") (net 8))
 (segment (start 124.974 71.054) (end 126.15 72.23) (width 0.25) (layer "B.Cu") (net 21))
 (segment (start 108.5 78.5) (end 107.194 77.194) (width 0.25) (layer "B.Cu") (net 21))
 (segment (start 107.194 71.742884) (end 107.882884 71.054) (width 0.25) (layer "B.Cu") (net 21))
 (segment (start 107.194 77.194) (end 107.194 71.742884) (width 0.25) (layer "B.Cu") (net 21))
 (segment (start 107.882884 71.054) (end 124.974 71.054) (width 0.25) (layer "B.Cu") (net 21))
 (segment (start 109.864 79.676) (end 107.324 79.676) (width 0.25) (layer "B.Cu") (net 22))
 (segment (start 107.696074 70.603) (end 127.063 70.603) (width 0.25) (layer "B.Cu") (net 22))
 (segment (start 107.324 79.676) (end 106.743 79.095) (width 0.25) (layer "B.Cu") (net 22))
 (segment (start 106.743 71.556074) (end 107.696074 70.603) (width 0.25) (layer "B.Cu") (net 22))
 (segment (start 127.063 70.603) (end 128.69 72.23) (width 0.25) (layer "B.Cu") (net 22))
 (segment (start 106.743 79.095) (end 106.743 71.556074) (width 0.25) (layer "B.Cu") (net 22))
 (segment (start 111.04 78.5) (end 109.864 79.676) (width 0.25) (layer "B.Cu") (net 22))
 (via (at 134.39 80) (size 0.9) (drill 0.6) (layers "F.Cu" "B.Cu") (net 11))
 (segment (start 134.39 80) (end 134.39 79.995793) (width 0.5) (layer "B.Cu") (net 11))
 (segment (start 138.314793 76.071) (end 142.629 76.071) (width 0.5) (layer "B.Cu") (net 11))
 (segment (start 134.39 79.995793) (end 138.314793 76.071) (width 0.5) (layer "B.Cu") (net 11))
 (segment (start 142.629 76.071) (end 143.93 74.77) (width 0.5) (layer "B.Cu") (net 11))
 (segment (start 145 77.5) (end 145 80.5) (width 0.5) (layer "F.Cu") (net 13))
 (via (at 145 77.5) (size 0.9) (drill 0.6) (layers "F.Cu" "B.Cu") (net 13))
 (via (at 131.85 80) (size 0.9) (drill 0.6) (layers "F.Cu" "B.Cu") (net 13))
 (via (at 145 77.5) (size 0.9) (drill 0.6) (layers "F.Cu" "B.Cu") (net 13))
 (via (at 145 80.5) (size 0.9) (drill 0.6) (layers "F.Cu" "B.Cu") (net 13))
 (segment (start 131.85 80.004207) (end 133.447793 81.602) (width 0.5) (layer "B.Cu") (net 13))
 (segment (start 146.47 76.03) (end 145 77.5) (width 0.5) (layer "B.Cu") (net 13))
 (segment (start 146.47 74.77) (end 146.47 76.03) (width 0.5) (layer "B.Cu") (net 13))
 (segment (start 133.447793 81.602) (end 143.898 81.602) (width 0.5) (layer "B.Cu") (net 13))
 (segment (start 131.85 80) (end 131.85 80.004207) (width 0.5) (layer "B.Cu") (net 13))
 (segment (start 143.898 81.602) (end 145 80.5) (width 0.5) (layer "B.Cu") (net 13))
 (segment (start 157.806 77.194) (end 157.806 71.742884) (width 0.25) (layer "B.Cu") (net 19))
 (segment (start 157.117116 71.054) (end 147.646 71.054) (width 0.25) (layer "B.Cu") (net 19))
 (segment (start 157.806 71.742884) (end 157.117116 71.054) (width 0.25) (layer "B.Cu") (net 19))
 (segment (start 147.646 71.054) (end 146.47 72.23) (width 0.25) (layer "B.Cu") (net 19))
 (segment (start 156.5 78.5) (end 157.806 77.194) (width 0.25) (layer "B.Cu") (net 19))
 (via (at 133.12 80) (size 0.9) (drill 0.6) (layers "F.Cu" "B.Cu") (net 12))
 (segment (start 149.01 74.77) (end 142.879 80.901) (width 0.5) (layer "B.Cu") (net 12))
 (segment (start 134.016793 80.901) (end 133.12 80.004207) (width 0.5) (layer "B.Cu") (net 12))
 (segment (start 133.12 80.004207) (end 133.12 80) (width 0.5) (layer "B.Cu") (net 12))
 (segment (start 142.879 80.901) (end 134.016793 80.901) (width 0.5) (layer "B.Cu") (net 12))
 (segment (start 150.186 75.602884) (end 153.083116 78.5) (width 0.25) (layer "B.Cu") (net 20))
 (segment (start 153.083116 78.5) (end 153.96 78.5) (width 0.25) (layer "B.Cu") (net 20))
 (segment (start 151.55 72.23) (end 150.186 73.594) (width 0.25) (layer "B.Cu") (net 20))
 (segment (start 150.186 73.594) (end 150.186 75.602884) (width 0.25) (layer "B.Cu") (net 20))
 (segment (start 116.12 82) (end 116.12 86.922) (width 1) (layer "F.Cu") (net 6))
 (segment (start 106.819 79.728) (end 106.819 72.681) (width 1) (layer "F.Cu") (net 6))
 (segment (start 127.503 98.305) (end 139 98.305) (width 1) (layer "F.Cu") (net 6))
 (segment (start 107.5 80.051) (end 107.142 80.051) (width 1) (layer "F.Cu") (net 6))
 (segment (start 110.91 72.23) (end 108.37 72.23) (width 1) (layer "F.Cu") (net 6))
 (segment (start 128.195 98.305) (end 127.503 98.305) (width 1) (layer "F.Cu") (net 6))
 (segment (start 135.505 98.305) (end 139 98.305) (width 1) (layer "F.Cu") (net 6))
 (segment (start 116.12 78.5) (end 114.569 80.051) (width 1) (layer "F.Cu") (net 6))
 (segment (start 131.5 95) (end 128.195 98.305) (width 1) (layer "F.Cu") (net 6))
 (segment (start 114.569 80.051) (end 107.5 80.051) (width 1) (layer "F.Cu") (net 6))
 (segment (start 124.698 95.5) (end 123.349 94.151) (width 1) (layer "F.Cu") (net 6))
 (segment (start 109.249 80.051) (end 116.12 86.922) (width 1) (layer "F.Cu") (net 6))
 (segment (start 131 95.5) (end 124.698 95.5) (width 1) (layer "F.Cu") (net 6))
 (segment (start 107.27 72.23) (end 108.37 72.23) (width 1) (layer "F.Cu") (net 6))
 (segment (start 116.12 86.922) (end 123.349 94.151) (width 1) (layer "F.Cu") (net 6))
 (segment (start 131.85 93.7) (end 131.85 94.65) (width 1) (layer "F.Cu") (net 6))
 (segment (start 123.349 94.151) (end 127.503 98.305) (width 1) (layer "F.Cu") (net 6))
 (segment (start 116.12 81.602) (end 114.569 80.051) (width 1) (layer "F.Cu") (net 6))
 (segment (start 131.85 94.65) (end 135.505 98.305) (width 1) (layer "F.Cu") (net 6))
 (segment (start 145 93.5) (end 145 82.38) (width 1) (layer "F.Cu") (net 6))
 (segment (start 139 98.305) (end 147.875 98.305) (width 1) (layer "F.Cu") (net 6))
 (segment (start 106.819 72.681) (end 107.27 72.23) (width 1) (layer "F.Cu") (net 6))
 (segment (start 116.12 78.5) (end 116.12 82) (width 1) (layer "F.Cu") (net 6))
 (segment (start 145 82.38) (end 148.88 78.5) (width 1) (layer "F.Cu") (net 6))
 (segment (start 107.5 80.051) (end 109.249 80.051) (width 1) (layer "F.Cu") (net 6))
 (segment (start 107.142 80.051) (end 106.819 79.728) (width 1) (layer "F.Cu") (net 6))
 (segment (start 131.85 94.65) (end 131.5 95) (width 1) (layer "F.Cu") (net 6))
 (segment (start 131.5 95) (end 131 95.5) (width 1) (layer "F.Cu") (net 6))
 (segment (start 116.12 82) (end 116.12 81.602) (width 1) (layer "F.Cu") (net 6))
 (via (at 147.875 98.305) (size 0.9) (drill 0.6) (layers "F.Cu" "B.Cu") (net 6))
 (via (at 145 93.5) (size 0.9) (drill 0.6) (layers "F.Cu" "B.Cu") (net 6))
 (segment (start 147.875 98.305) (end 145 95.43) (width 1) (layer "B.Cu") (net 6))
 (segment (start 145 95.43) (end 145 93.5) (width 1) (layer "B.Cu") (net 6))
 (segment (start 135.66 78.15) (end 135.66 80) (width 1) (layer "F.Cu") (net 10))
 (segment (start 130.92 77) (end 134.51 77) (width 1) (layer "F.Cu") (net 10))
 (segment (start 128.69 74.77) (end 130.92 77) (width 1) (layer "F.Cu") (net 10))
 (segment (start 134.51 77) (end 135.66 78.15) (width 1) (layer "F.Cu") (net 10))
 (via (at 129.31 93.7) (size 0.9) (drill 0.6) (layers "F.Cu" "B.Cu") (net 4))
 (segment (start 117.2 93.7) (end 102 78.5) (width 1) (layer "B.Cu") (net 4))
 (segment (start 129.31 93.7) (end 117.2 93.7) (width 1) (layer "B.Cu") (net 4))
 (via (at 130.58 93.7) (size 0.9) (drill 0.6) (layers "F.Cu" "B.Cu") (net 5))
 (segment (start 104.5 78.54) (end 104.54 78.5) (width 1) (layer "B.Cu") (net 5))
 (segment (start 130.511 93.20253) (end 129.80747 92.499) (width 1) (layer "B.Cu") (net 5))
 (segment (start 117.69747 92.499) (end 104.5 79.30153) (width 1) (layer "B.Cu") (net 5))
 (segment (start 104.5 79.30153) (end 104.5 78.54) (width 1) (layer "B.Cu") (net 5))
 (segment (start 130.511 93.7) (end 130.511 93.20253) (width 1) (layer "B.Cu") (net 5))
 (segment (start 129.80747 92.499) (end 117.69747 92.499) (width 1) (layer "B.Cu") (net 5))
 (segment (start 130.58 93.7) (end 130.511 93.7) (width 1) (layer "B.Cu") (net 5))
 (via (at 129.31 80) (size 0.9) (drill 0.6) (layers "F.Cu" "B.Cu") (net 15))
 (segment (start 138.761 89.951) (end 129.31 80.5) (width 1) (layer "B.Cu") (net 15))
 (segment (start 160.46 78.5) (end 160.46 87.842026) (width 1) (layer "B.Cu") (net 15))
 (segment (start 158.351026 89.951) (end 138.761 89.951) (width 1) (layer "B.Cu") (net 15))
 (segment (start 160.46 87.842026) (end 158.351026 89.951) (width 1) (layer "B.Cu") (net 15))
 (segment (start 129.31 80.5) (end 129.31 80) (width 1) (layer "B.Cu") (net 15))
 (via (at 130.58 80) (size 0.9) (drill 0.6) (layers "F.Cu" "B.Cu") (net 14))
 (segment (start 138.26353 91.152) (end 158.848497 91.151999) (width 1) (layer "B.Cu") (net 14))
 (segment (start 163 87.000496) (end 163 78.5) (width 1) (layer "B.Cu") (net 14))
 (segment (start 128.81253 78.799) (end 128.109 79.50253) (width 1) (layer "B.Cu") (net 14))
 (segment (start 158.848497 91.151999) (end 163 87.000496) (width 1) (layer "B.Cu") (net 14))
 (segment (start 128.109 79.50253) (end 128.109001 80.997471) (width 1) (layer "B.Cu") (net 14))
 (segment (start 128.109001 80.997471) (end 138.26353 91.152) (width 1) (layer "B.Cu") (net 14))
 (segment (start 130.58 80) (end 130.58 79.57153) (width 1) (layer "B.Cu") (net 14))
 (segment (start 129.80747 78.799) (end 128.81253 78.799) (width 1) (layer "B.Cu") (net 14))
 (segment (start 130.58 79.57153) (end 129.80747 78.799) (width 1) (layer "B.Cu") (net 14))
 (segment (start 147.875 93.745) (end 147.875 90.625) (width 1) (layer "F.Cu") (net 18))
 (segment (start 147.875 90.625) (end 151 87.5) (width 1) (layer "F.Cu") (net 18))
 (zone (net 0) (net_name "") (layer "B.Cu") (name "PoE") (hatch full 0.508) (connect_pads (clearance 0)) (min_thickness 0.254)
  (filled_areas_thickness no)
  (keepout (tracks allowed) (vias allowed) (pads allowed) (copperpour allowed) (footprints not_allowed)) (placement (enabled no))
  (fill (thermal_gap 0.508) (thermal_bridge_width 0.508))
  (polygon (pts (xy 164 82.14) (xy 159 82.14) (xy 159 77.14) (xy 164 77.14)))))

